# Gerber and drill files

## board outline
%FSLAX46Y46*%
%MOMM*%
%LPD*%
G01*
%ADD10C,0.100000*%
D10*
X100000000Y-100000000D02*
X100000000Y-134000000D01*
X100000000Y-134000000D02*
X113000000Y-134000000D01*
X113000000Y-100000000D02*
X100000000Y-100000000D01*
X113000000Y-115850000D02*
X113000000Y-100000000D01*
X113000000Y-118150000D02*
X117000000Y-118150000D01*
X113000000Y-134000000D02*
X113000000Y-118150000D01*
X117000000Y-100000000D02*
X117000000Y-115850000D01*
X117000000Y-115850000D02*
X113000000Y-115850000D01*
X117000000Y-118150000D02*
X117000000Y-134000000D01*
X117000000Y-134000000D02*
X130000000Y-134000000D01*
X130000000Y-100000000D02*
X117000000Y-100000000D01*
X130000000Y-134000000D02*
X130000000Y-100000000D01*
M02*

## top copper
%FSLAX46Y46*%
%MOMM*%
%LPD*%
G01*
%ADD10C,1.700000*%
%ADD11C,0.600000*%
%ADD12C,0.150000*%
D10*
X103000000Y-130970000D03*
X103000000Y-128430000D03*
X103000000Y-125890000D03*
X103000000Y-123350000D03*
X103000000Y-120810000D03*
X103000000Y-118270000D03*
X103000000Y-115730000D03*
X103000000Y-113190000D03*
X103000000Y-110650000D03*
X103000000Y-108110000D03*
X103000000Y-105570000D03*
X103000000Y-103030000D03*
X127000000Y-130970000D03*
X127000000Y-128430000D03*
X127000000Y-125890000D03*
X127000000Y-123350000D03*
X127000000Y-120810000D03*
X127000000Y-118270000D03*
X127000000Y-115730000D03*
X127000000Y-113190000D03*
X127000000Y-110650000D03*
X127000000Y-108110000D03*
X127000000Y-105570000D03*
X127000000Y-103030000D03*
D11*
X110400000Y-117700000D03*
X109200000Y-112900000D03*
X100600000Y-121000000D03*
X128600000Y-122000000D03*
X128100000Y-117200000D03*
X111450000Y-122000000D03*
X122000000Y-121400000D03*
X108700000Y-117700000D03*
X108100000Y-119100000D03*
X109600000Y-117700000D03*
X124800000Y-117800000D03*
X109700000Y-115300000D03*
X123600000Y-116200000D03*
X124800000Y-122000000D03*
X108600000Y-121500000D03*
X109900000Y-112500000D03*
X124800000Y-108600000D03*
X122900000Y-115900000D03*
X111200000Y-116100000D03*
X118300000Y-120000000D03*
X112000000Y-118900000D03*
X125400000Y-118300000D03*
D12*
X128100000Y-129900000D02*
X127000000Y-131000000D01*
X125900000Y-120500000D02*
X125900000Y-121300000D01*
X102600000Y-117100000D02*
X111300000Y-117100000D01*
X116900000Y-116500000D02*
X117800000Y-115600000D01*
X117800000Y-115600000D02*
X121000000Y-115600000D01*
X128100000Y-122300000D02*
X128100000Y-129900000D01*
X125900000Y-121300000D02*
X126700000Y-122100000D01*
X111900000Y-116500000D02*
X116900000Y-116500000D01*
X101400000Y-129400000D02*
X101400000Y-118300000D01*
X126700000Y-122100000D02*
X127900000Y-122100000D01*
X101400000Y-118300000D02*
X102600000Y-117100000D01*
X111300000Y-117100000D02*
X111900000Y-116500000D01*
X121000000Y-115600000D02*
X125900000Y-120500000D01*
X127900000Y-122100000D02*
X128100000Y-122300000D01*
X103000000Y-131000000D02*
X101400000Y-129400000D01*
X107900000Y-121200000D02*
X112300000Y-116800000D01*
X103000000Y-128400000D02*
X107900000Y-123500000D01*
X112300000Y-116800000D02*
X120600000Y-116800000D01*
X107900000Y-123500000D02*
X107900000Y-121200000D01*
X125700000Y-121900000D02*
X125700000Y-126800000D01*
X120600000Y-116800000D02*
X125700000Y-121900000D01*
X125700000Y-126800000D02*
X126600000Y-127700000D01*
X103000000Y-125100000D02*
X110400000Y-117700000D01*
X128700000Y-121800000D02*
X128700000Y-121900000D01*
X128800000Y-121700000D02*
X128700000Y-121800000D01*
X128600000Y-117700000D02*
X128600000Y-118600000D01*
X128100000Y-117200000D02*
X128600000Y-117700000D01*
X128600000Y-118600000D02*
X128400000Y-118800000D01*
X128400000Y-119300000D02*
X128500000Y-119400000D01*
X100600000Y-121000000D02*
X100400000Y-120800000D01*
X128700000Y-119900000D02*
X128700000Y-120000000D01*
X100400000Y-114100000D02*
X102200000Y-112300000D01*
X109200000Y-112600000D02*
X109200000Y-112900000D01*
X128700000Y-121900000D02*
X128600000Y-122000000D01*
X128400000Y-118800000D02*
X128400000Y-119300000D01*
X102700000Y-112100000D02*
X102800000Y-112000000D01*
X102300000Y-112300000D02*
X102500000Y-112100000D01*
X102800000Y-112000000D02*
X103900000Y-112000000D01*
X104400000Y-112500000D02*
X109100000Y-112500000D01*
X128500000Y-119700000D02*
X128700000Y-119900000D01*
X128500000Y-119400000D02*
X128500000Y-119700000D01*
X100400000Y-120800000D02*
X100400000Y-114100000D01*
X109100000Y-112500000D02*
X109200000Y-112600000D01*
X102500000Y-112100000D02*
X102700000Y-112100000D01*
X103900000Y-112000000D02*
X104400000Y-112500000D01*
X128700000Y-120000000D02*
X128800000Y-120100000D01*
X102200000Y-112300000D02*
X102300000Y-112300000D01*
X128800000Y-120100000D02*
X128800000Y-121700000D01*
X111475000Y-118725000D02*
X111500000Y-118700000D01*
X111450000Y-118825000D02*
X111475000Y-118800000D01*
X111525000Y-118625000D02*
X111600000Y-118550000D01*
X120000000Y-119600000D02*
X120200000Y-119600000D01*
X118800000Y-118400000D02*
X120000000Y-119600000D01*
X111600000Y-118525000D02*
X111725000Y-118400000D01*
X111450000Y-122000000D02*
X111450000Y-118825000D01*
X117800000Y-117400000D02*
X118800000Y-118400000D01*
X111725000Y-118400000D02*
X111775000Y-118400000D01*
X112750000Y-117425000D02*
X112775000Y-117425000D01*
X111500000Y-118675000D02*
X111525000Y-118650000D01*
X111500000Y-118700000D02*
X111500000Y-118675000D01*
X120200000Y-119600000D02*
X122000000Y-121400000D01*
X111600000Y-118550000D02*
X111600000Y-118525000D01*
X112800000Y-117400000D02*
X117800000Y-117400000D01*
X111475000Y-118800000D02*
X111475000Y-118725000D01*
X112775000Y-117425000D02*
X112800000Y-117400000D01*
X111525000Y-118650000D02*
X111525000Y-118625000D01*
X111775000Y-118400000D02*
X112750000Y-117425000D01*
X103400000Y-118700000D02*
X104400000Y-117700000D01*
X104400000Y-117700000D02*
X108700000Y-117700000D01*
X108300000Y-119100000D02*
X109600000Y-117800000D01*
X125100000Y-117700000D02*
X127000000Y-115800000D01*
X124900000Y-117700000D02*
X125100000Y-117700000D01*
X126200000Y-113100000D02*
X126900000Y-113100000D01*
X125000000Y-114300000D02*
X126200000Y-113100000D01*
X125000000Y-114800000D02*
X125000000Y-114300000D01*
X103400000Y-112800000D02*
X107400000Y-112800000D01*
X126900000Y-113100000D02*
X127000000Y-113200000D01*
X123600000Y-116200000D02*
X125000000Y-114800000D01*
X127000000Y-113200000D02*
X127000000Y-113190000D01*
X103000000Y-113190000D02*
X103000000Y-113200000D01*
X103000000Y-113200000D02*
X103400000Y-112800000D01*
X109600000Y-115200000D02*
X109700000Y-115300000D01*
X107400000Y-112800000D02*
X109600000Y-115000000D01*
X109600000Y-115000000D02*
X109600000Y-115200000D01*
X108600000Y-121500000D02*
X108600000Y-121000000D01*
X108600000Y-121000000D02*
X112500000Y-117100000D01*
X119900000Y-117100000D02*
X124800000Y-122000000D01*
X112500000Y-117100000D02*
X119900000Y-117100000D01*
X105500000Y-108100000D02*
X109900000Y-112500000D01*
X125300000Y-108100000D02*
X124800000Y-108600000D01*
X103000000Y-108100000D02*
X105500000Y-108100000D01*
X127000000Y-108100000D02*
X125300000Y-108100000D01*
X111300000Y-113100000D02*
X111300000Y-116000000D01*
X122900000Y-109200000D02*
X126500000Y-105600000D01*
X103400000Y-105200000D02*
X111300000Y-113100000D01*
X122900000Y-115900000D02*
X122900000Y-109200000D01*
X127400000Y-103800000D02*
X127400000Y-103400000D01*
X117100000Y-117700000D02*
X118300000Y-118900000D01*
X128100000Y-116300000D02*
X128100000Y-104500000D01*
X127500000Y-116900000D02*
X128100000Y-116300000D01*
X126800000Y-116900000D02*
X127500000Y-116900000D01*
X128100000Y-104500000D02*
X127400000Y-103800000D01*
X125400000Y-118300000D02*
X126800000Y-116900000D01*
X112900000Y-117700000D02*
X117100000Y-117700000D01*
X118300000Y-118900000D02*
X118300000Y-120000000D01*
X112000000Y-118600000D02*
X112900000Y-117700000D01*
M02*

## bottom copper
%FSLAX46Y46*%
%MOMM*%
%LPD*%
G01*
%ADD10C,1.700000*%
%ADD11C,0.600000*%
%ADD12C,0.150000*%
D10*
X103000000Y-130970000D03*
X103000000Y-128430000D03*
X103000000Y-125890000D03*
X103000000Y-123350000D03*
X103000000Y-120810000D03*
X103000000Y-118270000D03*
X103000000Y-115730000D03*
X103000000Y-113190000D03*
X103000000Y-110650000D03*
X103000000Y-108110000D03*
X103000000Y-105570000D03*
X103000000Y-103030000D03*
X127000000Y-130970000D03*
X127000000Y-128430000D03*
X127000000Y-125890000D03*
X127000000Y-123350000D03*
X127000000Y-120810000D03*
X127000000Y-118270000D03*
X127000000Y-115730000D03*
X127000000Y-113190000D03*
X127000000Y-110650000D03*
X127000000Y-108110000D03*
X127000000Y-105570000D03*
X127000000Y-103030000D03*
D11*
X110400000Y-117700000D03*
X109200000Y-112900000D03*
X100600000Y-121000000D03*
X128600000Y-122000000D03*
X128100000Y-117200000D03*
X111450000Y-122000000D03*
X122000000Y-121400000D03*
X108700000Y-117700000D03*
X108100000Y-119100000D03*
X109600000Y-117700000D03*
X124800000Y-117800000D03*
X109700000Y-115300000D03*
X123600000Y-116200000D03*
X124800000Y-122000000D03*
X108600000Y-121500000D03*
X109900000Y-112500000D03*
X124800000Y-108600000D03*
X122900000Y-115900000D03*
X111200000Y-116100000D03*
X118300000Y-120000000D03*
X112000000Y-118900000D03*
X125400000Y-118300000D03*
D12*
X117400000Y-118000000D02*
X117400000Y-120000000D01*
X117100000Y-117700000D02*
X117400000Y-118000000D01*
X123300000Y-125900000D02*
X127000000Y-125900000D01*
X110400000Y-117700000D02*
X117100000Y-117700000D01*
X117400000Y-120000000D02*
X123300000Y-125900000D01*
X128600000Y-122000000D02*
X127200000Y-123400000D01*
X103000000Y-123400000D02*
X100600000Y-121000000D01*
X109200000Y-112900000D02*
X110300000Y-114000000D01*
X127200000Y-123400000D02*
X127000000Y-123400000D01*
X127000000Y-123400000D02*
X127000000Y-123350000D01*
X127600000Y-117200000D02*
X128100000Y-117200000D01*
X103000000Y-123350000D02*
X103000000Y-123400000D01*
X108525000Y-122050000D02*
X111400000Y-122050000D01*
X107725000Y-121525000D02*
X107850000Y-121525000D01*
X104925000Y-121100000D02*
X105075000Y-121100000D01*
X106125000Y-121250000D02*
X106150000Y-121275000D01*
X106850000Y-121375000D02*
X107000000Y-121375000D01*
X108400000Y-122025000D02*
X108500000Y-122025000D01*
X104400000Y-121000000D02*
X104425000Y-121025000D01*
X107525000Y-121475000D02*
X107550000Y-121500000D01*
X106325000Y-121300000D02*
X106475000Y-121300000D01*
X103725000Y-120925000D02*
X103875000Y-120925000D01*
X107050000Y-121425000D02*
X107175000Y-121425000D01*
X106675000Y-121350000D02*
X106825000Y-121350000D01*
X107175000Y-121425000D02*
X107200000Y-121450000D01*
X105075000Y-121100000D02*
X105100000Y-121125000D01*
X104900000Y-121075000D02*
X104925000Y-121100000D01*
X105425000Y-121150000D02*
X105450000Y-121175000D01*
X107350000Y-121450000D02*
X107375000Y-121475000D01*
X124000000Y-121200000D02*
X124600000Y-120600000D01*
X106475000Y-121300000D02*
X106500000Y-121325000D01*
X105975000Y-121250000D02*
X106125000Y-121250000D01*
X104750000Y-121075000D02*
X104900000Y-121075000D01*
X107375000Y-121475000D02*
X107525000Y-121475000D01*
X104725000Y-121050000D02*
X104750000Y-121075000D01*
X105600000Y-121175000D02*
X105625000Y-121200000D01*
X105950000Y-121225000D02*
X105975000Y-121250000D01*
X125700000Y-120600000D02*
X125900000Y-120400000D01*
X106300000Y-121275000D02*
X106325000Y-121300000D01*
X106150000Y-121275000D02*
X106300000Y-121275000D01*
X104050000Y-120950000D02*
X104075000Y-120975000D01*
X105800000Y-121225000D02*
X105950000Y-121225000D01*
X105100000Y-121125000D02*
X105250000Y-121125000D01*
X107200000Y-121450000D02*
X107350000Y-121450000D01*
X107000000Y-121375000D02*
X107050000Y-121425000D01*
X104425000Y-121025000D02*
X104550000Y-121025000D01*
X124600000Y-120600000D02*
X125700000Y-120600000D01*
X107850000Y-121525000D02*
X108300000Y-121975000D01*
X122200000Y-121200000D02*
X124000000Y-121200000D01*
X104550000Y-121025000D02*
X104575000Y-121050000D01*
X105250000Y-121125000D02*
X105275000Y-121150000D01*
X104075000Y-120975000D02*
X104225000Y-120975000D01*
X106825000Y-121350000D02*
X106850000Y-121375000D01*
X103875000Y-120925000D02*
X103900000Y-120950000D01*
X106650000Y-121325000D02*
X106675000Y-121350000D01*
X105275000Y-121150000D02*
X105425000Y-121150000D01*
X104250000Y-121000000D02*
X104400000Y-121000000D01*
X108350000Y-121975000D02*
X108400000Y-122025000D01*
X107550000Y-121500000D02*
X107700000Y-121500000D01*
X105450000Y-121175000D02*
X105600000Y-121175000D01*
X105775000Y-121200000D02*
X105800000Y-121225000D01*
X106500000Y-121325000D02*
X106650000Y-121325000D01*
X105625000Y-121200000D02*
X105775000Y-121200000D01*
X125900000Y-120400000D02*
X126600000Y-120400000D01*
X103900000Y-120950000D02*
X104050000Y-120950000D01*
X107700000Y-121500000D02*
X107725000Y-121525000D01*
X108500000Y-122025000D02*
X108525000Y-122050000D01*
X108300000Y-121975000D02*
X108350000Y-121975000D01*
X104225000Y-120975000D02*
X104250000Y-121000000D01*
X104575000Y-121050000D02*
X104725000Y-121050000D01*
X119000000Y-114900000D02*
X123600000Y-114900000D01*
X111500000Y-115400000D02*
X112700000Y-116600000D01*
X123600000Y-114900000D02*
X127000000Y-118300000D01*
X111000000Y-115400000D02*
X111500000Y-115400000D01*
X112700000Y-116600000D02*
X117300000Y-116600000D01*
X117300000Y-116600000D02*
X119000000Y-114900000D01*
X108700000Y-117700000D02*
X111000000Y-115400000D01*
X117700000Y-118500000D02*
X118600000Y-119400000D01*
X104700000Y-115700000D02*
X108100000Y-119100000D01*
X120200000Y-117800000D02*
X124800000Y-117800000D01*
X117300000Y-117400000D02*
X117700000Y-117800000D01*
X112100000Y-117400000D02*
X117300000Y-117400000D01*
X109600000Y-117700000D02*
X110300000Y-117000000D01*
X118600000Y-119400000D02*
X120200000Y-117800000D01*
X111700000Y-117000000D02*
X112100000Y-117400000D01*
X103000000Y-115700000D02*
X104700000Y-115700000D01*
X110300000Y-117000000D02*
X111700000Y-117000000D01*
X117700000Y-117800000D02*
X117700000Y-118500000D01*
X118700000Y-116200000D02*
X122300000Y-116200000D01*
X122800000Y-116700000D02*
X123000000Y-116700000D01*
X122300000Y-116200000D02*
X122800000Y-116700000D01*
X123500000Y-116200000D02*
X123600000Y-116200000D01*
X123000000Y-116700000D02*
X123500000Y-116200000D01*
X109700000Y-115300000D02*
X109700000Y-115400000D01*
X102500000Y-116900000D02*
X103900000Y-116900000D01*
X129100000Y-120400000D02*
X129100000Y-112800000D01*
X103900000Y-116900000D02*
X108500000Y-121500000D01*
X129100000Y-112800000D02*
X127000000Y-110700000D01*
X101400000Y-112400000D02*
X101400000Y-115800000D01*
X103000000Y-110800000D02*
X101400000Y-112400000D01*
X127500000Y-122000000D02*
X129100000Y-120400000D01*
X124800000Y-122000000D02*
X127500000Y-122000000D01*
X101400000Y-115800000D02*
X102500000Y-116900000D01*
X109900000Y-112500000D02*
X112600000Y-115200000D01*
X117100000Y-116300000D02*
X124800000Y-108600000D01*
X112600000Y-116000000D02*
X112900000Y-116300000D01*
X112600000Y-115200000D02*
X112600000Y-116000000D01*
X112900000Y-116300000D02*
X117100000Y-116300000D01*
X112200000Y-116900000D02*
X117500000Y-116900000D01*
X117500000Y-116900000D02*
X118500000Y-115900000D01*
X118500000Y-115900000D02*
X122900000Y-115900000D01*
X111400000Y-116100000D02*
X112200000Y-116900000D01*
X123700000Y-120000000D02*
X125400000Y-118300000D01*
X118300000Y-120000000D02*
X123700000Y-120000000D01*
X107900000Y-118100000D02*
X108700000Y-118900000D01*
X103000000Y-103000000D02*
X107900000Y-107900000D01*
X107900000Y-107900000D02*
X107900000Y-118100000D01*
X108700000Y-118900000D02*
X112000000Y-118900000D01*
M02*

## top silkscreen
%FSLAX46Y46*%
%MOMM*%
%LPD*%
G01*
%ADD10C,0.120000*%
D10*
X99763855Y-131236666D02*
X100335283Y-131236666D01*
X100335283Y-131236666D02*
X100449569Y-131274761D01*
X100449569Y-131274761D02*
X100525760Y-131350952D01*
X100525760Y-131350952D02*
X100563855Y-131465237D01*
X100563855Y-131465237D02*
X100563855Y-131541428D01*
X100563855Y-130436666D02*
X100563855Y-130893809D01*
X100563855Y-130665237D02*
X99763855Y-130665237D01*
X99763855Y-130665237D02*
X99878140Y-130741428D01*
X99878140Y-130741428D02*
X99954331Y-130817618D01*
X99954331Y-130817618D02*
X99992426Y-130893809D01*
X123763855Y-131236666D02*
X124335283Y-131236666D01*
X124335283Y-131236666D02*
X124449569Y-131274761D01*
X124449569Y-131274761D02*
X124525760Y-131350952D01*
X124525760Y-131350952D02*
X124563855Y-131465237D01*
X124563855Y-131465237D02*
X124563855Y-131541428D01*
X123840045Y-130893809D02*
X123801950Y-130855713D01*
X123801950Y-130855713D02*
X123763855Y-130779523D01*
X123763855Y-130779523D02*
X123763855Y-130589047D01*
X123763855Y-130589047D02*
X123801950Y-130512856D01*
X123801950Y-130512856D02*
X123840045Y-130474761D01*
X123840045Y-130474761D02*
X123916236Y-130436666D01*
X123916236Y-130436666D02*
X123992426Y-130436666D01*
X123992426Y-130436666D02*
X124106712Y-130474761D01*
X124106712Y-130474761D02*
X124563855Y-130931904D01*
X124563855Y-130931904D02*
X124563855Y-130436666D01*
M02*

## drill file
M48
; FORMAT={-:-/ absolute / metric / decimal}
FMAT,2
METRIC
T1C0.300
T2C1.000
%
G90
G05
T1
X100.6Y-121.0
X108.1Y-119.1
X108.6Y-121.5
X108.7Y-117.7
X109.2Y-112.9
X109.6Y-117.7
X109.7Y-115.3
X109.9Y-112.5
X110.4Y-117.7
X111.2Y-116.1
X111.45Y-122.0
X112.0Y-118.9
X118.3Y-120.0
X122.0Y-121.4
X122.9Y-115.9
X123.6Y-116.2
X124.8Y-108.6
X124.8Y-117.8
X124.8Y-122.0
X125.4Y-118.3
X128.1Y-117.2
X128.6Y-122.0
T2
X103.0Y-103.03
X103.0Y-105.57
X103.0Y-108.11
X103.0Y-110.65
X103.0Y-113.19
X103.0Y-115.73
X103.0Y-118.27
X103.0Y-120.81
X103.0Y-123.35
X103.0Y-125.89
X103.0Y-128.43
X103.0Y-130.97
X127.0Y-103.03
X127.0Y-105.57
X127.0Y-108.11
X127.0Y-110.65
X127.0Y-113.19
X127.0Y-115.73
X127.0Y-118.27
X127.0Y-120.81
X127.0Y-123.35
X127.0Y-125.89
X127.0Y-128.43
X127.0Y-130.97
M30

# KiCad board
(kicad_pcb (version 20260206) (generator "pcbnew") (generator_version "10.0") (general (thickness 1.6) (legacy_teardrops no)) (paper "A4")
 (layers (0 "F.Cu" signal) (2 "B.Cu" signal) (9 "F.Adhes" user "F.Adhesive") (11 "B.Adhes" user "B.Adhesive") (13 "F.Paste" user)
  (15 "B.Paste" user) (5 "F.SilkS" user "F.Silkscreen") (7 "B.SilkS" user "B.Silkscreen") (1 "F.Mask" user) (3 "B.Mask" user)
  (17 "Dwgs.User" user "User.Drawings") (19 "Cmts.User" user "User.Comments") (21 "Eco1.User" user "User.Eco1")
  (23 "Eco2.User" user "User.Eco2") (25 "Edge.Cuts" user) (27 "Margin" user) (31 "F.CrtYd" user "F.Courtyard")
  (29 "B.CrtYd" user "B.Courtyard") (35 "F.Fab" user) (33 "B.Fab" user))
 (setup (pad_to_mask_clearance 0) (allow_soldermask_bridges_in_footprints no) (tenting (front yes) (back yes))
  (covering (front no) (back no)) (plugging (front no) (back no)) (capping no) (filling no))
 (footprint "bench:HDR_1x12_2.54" (layer "F.Cu") (at 103 130.97 90)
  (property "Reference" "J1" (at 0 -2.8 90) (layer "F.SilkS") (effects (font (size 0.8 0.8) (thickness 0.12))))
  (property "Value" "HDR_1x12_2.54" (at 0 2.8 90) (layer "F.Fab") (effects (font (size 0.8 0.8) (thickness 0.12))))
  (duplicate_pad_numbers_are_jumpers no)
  (pad "1" thru_hole circle (at 0 0 90) (size 1.7 1.7) (drill 1) (layers "*.Cu" "*.Mask") (remove_unused_layers no) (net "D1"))
  (pad "2" thru_hole circle (at 2.54 0 90) (size 1.7 1.7) (drill 1) (layers "*.Cu" "*.Mask") (remove_unused_layers no) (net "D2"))
  (pad "3" thru_hole circle (at 5.08 0 90) (size 1.7 1.7) (drill 1) (layers "*.Cu" "*.Mask") (remove_unused_layers no) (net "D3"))
  (pad "4" thru_hole circle (at 7.62 0 90) (size 1.7 1.7) (drill 1) (layers "*.Cu" "*.Mask") (remove_unused_layers no) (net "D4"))
  (pad "5" thru_hole circle (at 10.16 0 90) (size 1.7 1.7) (drill 1) (layers "*.Cu" "*.Mask") (remove_unused_layers no) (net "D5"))
  (pad "6" thru_hole circle (at 12.7 0 90) (size 1.7 1.7) (drill 1) (layers "*.Cu" "*.Mask") (remove_unused_layers no) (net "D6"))
  (pad "7" thru_hole circle (at 15.24 0 90) (size 1.7 1.7) (drill 1) (layers "*.Cu" "*.Mask") (remove_unused_layers no) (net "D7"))
  (pad "8" thru_hole circle (at 17.78 0 90) (size 1.7 1.7) (drill 1) (layers "*.Cu" "*.Mask") (remove_unused_layers no) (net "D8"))
  (pad "9" thru_hole circle (at 20.32 0 90) (size 1.7 1.7) (drill 1) (layers "*.Cu" "*.Mask") (remove_unused_layers no) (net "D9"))
  (pad "10" thru_hole circle (at 22.86 0 90) (size 1.7 1.7) (drill 1) (layers "*.Cu" "*.Mask") (remove_unused_layers no) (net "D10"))
  (pad "11" thru_hole circle (at 25.4 0 90) (size 1.7 1.7) (drill 1) (layers "*.Cu" "*.Mask") (remove_unused_layers no) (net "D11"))
  (pad "12" thru_hole circle (at 27.94 0 90) (size 1.7 1.7) (drill 1) (layers "*.Cu" "*.Mask") (remove_unused_layers no) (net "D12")))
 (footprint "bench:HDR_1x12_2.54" (layer "F.Cu") (at 127 130.97 90)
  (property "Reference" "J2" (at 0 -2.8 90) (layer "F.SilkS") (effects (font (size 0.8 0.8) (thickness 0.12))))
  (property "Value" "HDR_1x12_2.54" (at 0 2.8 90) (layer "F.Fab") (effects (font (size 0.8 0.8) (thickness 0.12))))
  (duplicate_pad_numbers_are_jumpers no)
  (pad "1" thru_hole circle (at 0 0 90) (size 1.7 1.7) (drill 1) (layers "*.Cu" "*.Mask") (remove_unused_layers no) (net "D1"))
  (pad "2" thru_hole circle (at 2.54 0 90) (size 1.7 1.7) (drill 1) (layers "*.Cu" "*.Mask") (remove_unused_layers no) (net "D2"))
  (pad "3" thru_hole circle (at 5.08 0 90) (size 1.7 1.7) (drill 1) (layers "*.Cu" "*.Mask") (remove_unused_layers no) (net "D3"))
  (pad "4" thru_hole circle (at 7.62 0 90) (size 1.7 1.7) (drill 1) (layers "*.Cu" "*.Mask") (remove_unused_layers no) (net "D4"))
  (pad "5" thru_hole circle (at 10.16 0 90) (size 1.7 1.7) (drill 1) (layers "*.Cu" "*.Mask") (remove_unused_layers no) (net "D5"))
  (pad "6" thru_hole circle (at 12.7 0 90) (size 1.7 1.7) (drill 1) (layers "*.Cu" "*.Mask") (remove_unused_layers no) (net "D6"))
  (pad "7" thru_hole circle (at 15.24 0 90) (size 1.7 1.7) (drill 1) (layers "*.Cu" "*.Mask") (remove_unused_layers no) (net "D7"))
  (pad "8" thru_hole circle (at 17.78 0 90) (size 1.7 1.7) (drill 1) (layers "*.Cu" "*.Mask") (remove_unused_layers no) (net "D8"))
  (pad "9" thru_hole circle (at 20.32 0 90) (size 1.7 1.7) (drill 1) (layers "*.Cu" "*.Mask") (remove_unused_layers no) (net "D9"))
  (pad "10" thru_hole circle (at 22.86 0 90) (size 1.7 1.7) (drill 1) (layers "*.Cu" "*.Mask") (remove_unused_layers no) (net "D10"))
  (pad "11" thru_hole circle (at 25.4 0 90) (size 1.7 1.7) (drill 1) (layers "*.Cu" "*.Mask") (remove_unused_layers no) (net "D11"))
  (pad "12" thru_hole circle (at 27.94 0 90) (size 1.7 1.7) (drill 1) (layers "*.Cu" "*.Mask") (remove_unused_layers no) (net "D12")))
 (gr_line (start 100 100) (end 100 134) (stroke (width 0.1) (type solid)) (layer "Edge.Cuts"))
 (gr_line (start 100 134) (end 113 134) (stroke (width 0.1) (type solid)) (layer "Edge.Cuts"))
 (gr_line (start 113 100) (end 100 100) (stroke (width 0.1) (type solid)) (layer "Edge.Cuts"))
 (gr_line (start 113 115.85) (end 113 100) (stroke (width 0.1) (type solid)) (layer "Edge.Cuts"))
 (gr_line (start 113 118.15) (end 117 118.15) (stroke (width 0.1) (type solid)) (layer "Edge.Cuts"))
 (gr_line (start 113 134) (end 113 118.15) (stroke (width 0.1) (type solid)) (layer "Edge.Cuts"))
 (gr_line (start 117 100) (end 117 115.85) (stroke (width 0.1) (type solid)) (layer "Edge.Cuts"))
 (gr_line (start 117 115.85) (end 113 115.85) (stroke (width 0.1) (type solid)) (layer "Edge.Cuts"))
 (gr_line (start 117 118.15) (end 117 134) (stroke (width 0.1) (type solid)) (layer "Edge.Cuts"))
 (gr_line (start 117 134) (end 130 134) (stroke (width 0.1) (type solid)) (layer "Edge.Cuts"))
 (gr_line (start 130 100) (end 117 100) (stroke (width 0.1) (type solid)) (layer "Edge.Cuts"))
 (gr_line (start 130 134) (end 130 100) (stroke (width 0.1) (type solid)) (layer "Edge.Cuts"))
 (segment (start 128.1 129.9) (end 127 131) (width 0.15) (layer "F.Cu") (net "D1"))
 (segment (start 125.9 120.5) (end 125.9 121.3) (width 0.15) (layer "F.Cu") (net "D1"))
 (segment (start 102.6 117.1) (end 111.3 117.1) (width 0.15) (layer "F.Cu") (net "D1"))
 (segment (start 116.9 116.5) (end 117.8 115.6) (width 0.15) (layer "F.Cu") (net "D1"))
 (segment (start 117.8 115.6) (end 121 115.6) (width 0.15) (layer "F.Cu") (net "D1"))
 (segment (start 128.1 122.3) (end 128.1 129.9) (width 0.15) (layer "F.Cu") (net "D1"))
 (segment (start 125.9 121.3) (end 126.7 122.1) (width 0.15) (layer "F.Cu") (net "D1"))
 (segment (start 111.9 116.5) (end 116.9 116.5) (width 0.15) (layer "F.Cu") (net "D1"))
 (segment (start 101.4 129.4) (end 101.4 118.3) (width 0.15) (layer "F.Cu") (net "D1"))
 (segment (start 126.7 122.1) (end 127.9 122.1) (width 0.15) (layer "F.Cu") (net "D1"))
 (segment (start 101.4 118.3) (end 102.6 117.1) (width 0.15) (layer "F.Cu") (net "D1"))
 (segment (start 111.3 117.1) (end 111.9 116.5) (width 0.15) (layer "F.Cu") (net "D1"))
 (segment (start 121 115.6) (end 125.9 120.5) (width 0.15) (layer "F.Cu") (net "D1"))
 (segment (start 127.9 122.1) (end 128.1 122.3) (width 0.15) (layer "F.Cu") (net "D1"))
 (segment (start 103 131) (end 101.4 129.4) (width 0.15) (layer "F.Cu") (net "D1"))
 (segment (start 107.9 121.2) (end 112.3 116.8) (width 0.15) (layer "F.Cu") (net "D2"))
 (segment (start 103 128.4) (end 107.9 123.5) (width 0.15) (layer "F.Cu") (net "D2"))
 (segment (start 112.3 116.8) (end 120.6 116.8) (width 0.15) (layer "F.Cu") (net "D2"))
 (segment (start 107.9 123.5) (end 107.9 121.2) (width 0.15) (layer "F.Cu") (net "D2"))
 (segment (start 125.7 121.9) (end 125.7 126.8) (width 0.15) (layer "F.Cu") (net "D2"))
 (segment (start 120.6 116.8) (end 125.7 121.9) (width 0.15) (layer "F.Cu") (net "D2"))
 (segment (start 125.7 126.8) (end 126.6 127.7) (width 0.15) (layer "F.Cu") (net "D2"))
 (segment (start 103 125.1) (end 110.4 117.7) (width 0.15) (layer "F.Cu") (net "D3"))
 (via (at 110.4 117.7) (size 0.6) (drill 0.3) (layers "F.Cu" "B.Cu") (capping no) (covering (front no) (back no))
  (plugging (front no) (back no)) (filling no) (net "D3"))
 (segment (start 117.4 118) (end 117.4 120) (width 0.15) (layer "B.Cu") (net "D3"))
 (segment (start 117.1 117.7) (end 117.4 118) (width 0.15) (layer "B.Cu") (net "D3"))
 (segment (start 123.3 125.9) (end 127 125.9) (width 0.15) (layer "B.Cu") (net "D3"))
 (segment (start 110.4 117.7) (end 117.1 117.7) (width 0.15) (layer "B.Cu") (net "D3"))
 (segment (start 117.4 120) (end 123.3 125.9) (width 0.15) (layer "B.Cu") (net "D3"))
 (segment (start 128.7 121.8) (end 128.7 121.9) (width 0.15) (layer "F.Cu") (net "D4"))
 (segment (start 128.8 121.7) (end 128.7 121.8) (width 0.15) (layer "F.Cu") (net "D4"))
 (segment (start 128.6 117.7) (end 128.6 118.6) (width 0.15) (layer "F.Cu") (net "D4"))
 (segment (start 128.1 117.2) (end 128.6 117.7) (width 0.15) (layer "F.Cu") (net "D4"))
 (segment (start 128.6 118.6) (end 128.4 118.8) (width 0.15) (layer "F.Cu") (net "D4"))
 (segment (start 128.4 119.3) (end 128.5 119.4) (width 0.15) (layer "F.Cu") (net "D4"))
 (segment (start 100.6 121) (end 100.4 120.8) (width 0.15) (layer "F.Cu") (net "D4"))
 (segment (start 128.7 119.9) (end 128.7 120) (width 0.15) (layer "F.Cu") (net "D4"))
 (segment (start 100.4 114.1) (end 102.2 112.3) (width 0.15) (layer "F.Cu") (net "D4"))
 (segment (start 109.2 112.6) (end 109.2 112.9) (width 0.15) (layer "F.Cu") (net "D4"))
 (segment (start 128.7 121.9) (end 128.6 122) (width 0.15) (layer "F.Cu") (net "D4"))
 (segment (start 128.4 118.8) (end 128.4 119.3) (width 0.15) (layer "F.Cu") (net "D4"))
 (segment (start 102.7 112.1) (end 102.8 112) (width 0.15) (layer "F.Cu") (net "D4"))
 (segment (start 102.3 112.3) (end 102.5 112.1) (width 0.15) (layer "F.Cu") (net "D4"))
 (segment (start 102.8 112) (end 103.9 112) (width 0.15) (layer "F.Cu") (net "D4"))
 (segment (start 104.4 112.5) (end 109.1 112.5) (width 0.15) (layer "F.Cu") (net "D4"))
 (segment (start 128.5 119.7) (end 128.7 119.9) (width 0.15) (layer "F.Cu") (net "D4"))
 (segment (start 128.5 119.4) (end 128.5 119.7) (width 0.15) (layer "F.Cu") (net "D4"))
 (segment (start 100.4 120.8) (end 100.4 114.1) (width 0.15) (layer "F.Cu") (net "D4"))
 (segment (start 109.1 112.5) (end 109.2 112.6) (width 0.15) (layer "F.Cu") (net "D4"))
 (segment (start 102.5 112.1) (end 102.7 112.1) (width 0.15) (layer "F.Cu") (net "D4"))
 (segment (start 103.9 112) (end 104.4 112.5) (width 0.15) (layer "F.Cu") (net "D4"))
 (segment (start 128.7 120) (end 128.8 120.1) (width 0.15) (layer "F.Cu") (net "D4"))
 (segment (start 102.2 112.3) (end 102.3 112.3) (width 0.15) (layer "F.Cu") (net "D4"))
 (segment (start 128.8 120.1) (end 128.8 121.7) (width 0.15) (layer "F.Cu") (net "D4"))
 (via (at 109.2 112.9) (size 0.6) (drill 0.3) (layers "F.Cu" "B.Cu") (capping no) (covering (front no) (back no))
  (plugging (front no) (back no)) (filling no) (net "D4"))
 (via (at 100.6 121) (size 0.6) (drill 0.3) (layers "F.Cu" "B.Cu") (capping no) (covering (front no) (back no))
  (plugging (front no) (back no)) (filling no) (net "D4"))
 (via (at 128.6 122) (size 0.6) (drill 0.3) (layers "F.Cu" "B.Cu") (capping no) (covering (front no) (back no))
  (plugging (front no) (back no)) (filling no) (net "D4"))
 (via (at 128.1 117.2) (size 0.6) (drill 0.3) (layers "F.Cu" "B.Cu") (capping no) (covering (front no) (back no))
  (plugging (front no) (back no)) (filling no) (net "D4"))
 (segment (start 128.6 122) (end 127.2 123.4) (width 0.15) (layer "B.Cu") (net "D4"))
 (segment (start 103 123.4) (end 100.6 121) (width 0.15) (layer "B.Cu") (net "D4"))
 (segment (start 109.2 112.9) (end 110.3 114) (width 0.15) (layer "B.Cu") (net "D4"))
 (segment (start 127.2 123.4) (end 127 123.4) (width 0.15) (layer "B.Cu") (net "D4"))
 (segment (start 127 123.4) (end 127 123.35) (width 0.15) (layer "B.Cu") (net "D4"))
 (segment (start 127.6 117.2) (end 128.1 117.2) (width 0.15) (layer "B.Cu") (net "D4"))
 (segment (start 103 123.35) (end 103 123.4) (width 0.15) (layer "B.Cu") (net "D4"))
 (segment (start 111.475 118.725) (end 111.5 118.7) (width 0.15) (layer "F.Cu") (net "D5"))
 (segment (start 111.45 118.825) (end 111.475 118.8) (width 0.15) (layer "F.Cu") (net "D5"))
 (segment (start 111.525 118.625) (end 111.6 118.55) (width 0.15) (layer "F.Cu") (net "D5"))
 (segment (start 120 119.6) (end 120.2 119.6) (width 0.15) (layer "F.Cu") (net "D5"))
 (segment (start 118.8 118.4) (end 120 119.6) (width 0.15) (layer "F.Cu") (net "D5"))
 (segment (start 111.6 118.525) (end 111.725 118.4) (width 0.15) (layer "F.Cu") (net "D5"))
 (segment (start 111.45 122) (end 111.45 118.825) (width 0.15) (layer "F.Cu") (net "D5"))
 (segment (start 117.8 117.4) (end 118.8 118.4) (width 0.15) (layer "F.Cu") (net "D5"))
 (segment (start 111.725 118.4) (end 111.775 118.4) (width 0.15) (layer "F.Cu") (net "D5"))
 (segment (start 112.75 117.425) (end 112.775 117.425) (width 0.15) (layer "F.Cu") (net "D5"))
 (segment (start 111.5 118.675) (end 111.525 118.65) (width 0.15) (layer "F.Cu") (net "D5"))
 (segment (start 111.5 118.7) (end 111.5 118.675) (width 0.15) (layer "F.Cu") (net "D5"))
 (segment (start 120.2 119.6) (end 122 121.4) (width 0.15) (layer "F.Cu") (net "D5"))
 (segment (start 111.6 118.55) (end 111.6 118.525) (width 0.15) (layer "F.Cu") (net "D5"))
 (segment (start 112.8 117.4) (end 117.8 117.4) (width 0.15) (layer "F.Cu") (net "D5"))
 (segment (start 111.475 118.8) (end 111.475 118.725) (width 0.15) (layer "F.Cu") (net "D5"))
 (segment (start 112.775 117.425) (end 112.8 117.4) (width 0.15) (layer "F.Cu") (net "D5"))
 (segment (start 111.525 118.65) (end 111.525 118.625) (width 0.15) (layer "F.Cu") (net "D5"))
 (segment (start 111.775 118.4) (end 112.75 117.425) (width 0.15) (layer "F.Cu") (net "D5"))
 (via (at 111.45 122) (size 0.6) (drill 0.3) (layers "F.Cu" "B.Cu") (capping no) (covering (front no) (back no))
  (plugging (front no) (back no)) (filling no) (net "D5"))
 (via (at 122 121.4) (size 0.6) (drill 0.3) (layers "F.Cu" "B.Cu") (capping no) (covering (front no) (back no))
  (plugging (front no) (back no)) (filling no) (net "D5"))
 (segment (start 108.525 122.05) (end 111.4 122.05) (width 0.15) (layer "B.Cu") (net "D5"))
 (segment (start 107.725 121.525) (end 107.85 121.525) (width 0.15) (layer "B.Cu") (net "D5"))
 (segment (start 104.925 121.1) (end 105.075 121.1) (width 0.15) (layer "B.Cu") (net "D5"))
 (segment (start 106.125 121.25) (end 106.15 121.275) (width 0.15) (layer "B.Cu") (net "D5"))
 (segment (start 106.85 121.375) (end 107 121.375) (width 0.15) (layer "B.Cu") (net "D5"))
 (segment (start 108.4 122.025) (end 108.5 122.025) (width 0.15) (layer "B.Cu") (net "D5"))
 (segment (start 104.4 121) (end 104.425 121.025) (width 0.15) (layer "B.Cu") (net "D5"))
 (segment (start 107.525 121.475) (end 107.55 121.5) (width 0.15) (layer "B.Cu") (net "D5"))
 (segment (start 106.325 121.3) (end 106.475 121.3) (width 0.15) (layer "B.Cu") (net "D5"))
 (segment (start 103.725 120.925) (end 103.875 120.925) (width 0.15) (layer "B.Cu") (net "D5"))
 (segment (start 107.05 121.425) (end 107.175 121.425) (width 0.15) (layer "B.Cu") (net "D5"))
 (segment (start 106.675 121.35) (end 106.825 121.35) (width 0.15) (layer "B.Cu") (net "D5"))
 (segment (start 107.175 121.425) (end 107.2 121.45) (width 0.15) (layer "B.Cu") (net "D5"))
 (segment (start 105.075 121.1) (end 105.1 121.125) (width 0.15) (layer "B.Cu") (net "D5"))
 (segment (start 104.9 121.075) (end 104.925 121.1) (width 0.15) (layer "B.Cu") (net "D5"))
 (segment (start 105.425 121.15) (end 105.45 121.175) (width 0.15) (layer "B.Cu") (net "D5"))
 (segment (start 107.35 121.45) (end 107.375 121.475) (width 0.15) (layer "B.Cu") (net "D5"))
 (segment (start 124 121.2) (end 124.6 120.6) (width 0.15) (layer "B.Cu") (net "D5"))
 (segment (start 106.475 121.3) (end 106.5 121.325) (width 0.15) (layer "B.Cu") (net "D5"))
 (segment (start 105.975 121.25) (end 106.125 121.25) (width 0.15) (layer "B.Cu") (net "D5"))
 (segment (start 104.75 121.075) (end 104.9 121.075) (width 0.15) (layer "B.Cu") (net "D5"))
 (segment (start 107.375 121.475) (end 107.525 121.475) (width 0.15) (layer "B.Cu") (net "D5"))
 (segment (start 104.725 121.05) (end 104.75 121.075) (width 0.15) (layer "B.Cu") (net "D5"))
 (segment (start 105.6 121.175) (end 105.625 121.2) (width 0.15) (layer "B.Cu") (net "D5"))
 (segment (start 105.95 121.225) (end 105.975 121.25) (width 0.15) (layer "B.Cu") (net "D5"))
 (segment (start 125.7 120.6) (end 125.9 120.4) (width 0.15) (layer "B.Cu") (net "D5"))
 (segment (start 106.3 121.275) (end 106.325 121.3) (width 0.15) (layer "B.Cu") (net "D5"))
 (segment (start 106.15 121.275) (end 106.3 121.275) (width 0.15) (layer "B.Cu") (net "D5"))
 (segment (start 104.05 120.95) (end 104.075 120.975) (width 0.15) (layer "B.Cu") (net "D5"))
 (segment (start 105.8 121.225) (end 105.95 121.225) (width 0.15) (layer "B.Cu") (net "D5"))
 (segment (start 105.1 121.125) (end 105.25 121.125) (width 0.15) (layer "B.Cu") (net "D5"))
 (segment (start 107.2 121.45) (end 107.35 121.45) (width 0.15) (layer "B.Cu") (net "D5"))
 (segment (start 107 121.375) (end 107.05 121.425) (width 0.15) (layer "B.Cu") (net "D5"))
 (segment (start 104.425 121.025) (end 104.55 121.025) (width 0.15) (layer "B.Cu") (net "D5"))
 (segment (start 124.6 120.6) (end 125.7 120.6) (width 0.15) (layer "B.Cu") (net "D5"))
 (segment (start 107.85 121.525) (end 108.3 121.975) (width 0.15) (layer "B.Cu") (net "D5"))
 (segment (start 122.2 121.2) (end 124 121.2) (width 0.15) (layer "B.Cu") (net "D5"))
 (segment (start 104.55 121.025) (end 104.575 121.05) (width 0.15) (layer "B.Cu") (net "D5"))
 (segment (start 105.25 121.125) (end 105.275 121.15) (width 0.15) (layer "B.Cu") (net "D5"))
 (segment (start 104.075 120.975) (end 104.225 120.975) (width 0.15) (layer "B.Cu") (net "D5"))
 (segment (start 106.825 121.35) (end 106.85 121.375) (width 0.15) (layer "B.Cu") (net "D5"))
 (segment (start 103.875 120.925) (end 103.9 120.95) (width 0.15) (layer "B.Cu") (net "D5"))
 (segment (start 106.65 121.325) (end 106.675 121.35) (width 0.15) (layer "B.Cu") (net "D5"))
 (segment (start 105.275 121.15) (end 105.425 121.15) (width 0.15) (layer "B.Cu") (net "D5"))
 (segment (start 104.25 121) (end 104.4 121) (width 0.15) (layer "B.Cu") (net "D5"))
 (segment (start 108.35 121.975) (end 108.4 122.025) (width 0.15) (layer "B.Cu") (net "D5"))
 (segment (start 107.55 121.5) (end 107.7 121.5) (width 0.15) (layer "B.Cu") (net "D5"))
 (segment (start 105.45 121.175) (end 105.6 121.175) (width 0.15) (layer "B.Cu") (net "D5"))
 (segment (start 105.775 121.2) (end 105.8 121.225) (width 0.15) (layer "B.Cu") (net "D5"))
 (segment (start 106.5 121.325) (end 106.65 121.325) (width 0.15) (layer "B.Cu") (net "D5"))
 (segment (start 105.625 121.2) (end 105.775 121.2) (width 0.15) (layer "B.Cu") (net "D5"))
 (segment (start 125.9 120.4) (end 126.6 120.4) (width 0.15) (layer "B.Cu") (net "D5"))
 (segment (start 103.9 120.95) (end 104.05 120.95) (width 0.15) (layer "B.Cu") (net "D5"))
 (segment (start 107.7 121.5) (end 107.725 121.525) (width 0.15) (layer "B.Cu") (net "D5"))
 (segment (start 108.5 122.025) (end 108.525 122.05) (width 0.15) (layer "B.Cu") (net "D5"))
 (segment (start 108.3 121.975) (end 108.35 121.975) (width 0.15) (layer "B.Cu") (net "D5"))
 (segment (start 104.225 120.975) (end 104.25 121) (width 0.15) (layer "B.Cu") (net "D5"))
 (segment (start 104.575 121.05) (end 104.725 121.05) (width 0.15) (layer "B.Cu") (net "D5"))
 (segment (start 103.4 118.7) (end 104.4 117.7) (width 0.15) (layer "F.Cu") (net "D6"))
 (segment (start 104.4 117.7) (end 108.7 117.7) (width 0.15) (layer "F.Cu") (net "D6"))
 (via (at 108.7 117.7) (size 0.6) (drill 0.3) (layers "F.Cu" "B.Cu") (capping no) (covering (front no) (back no))
  (plugging (front no) (back no)) (filling no) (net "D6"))
 (segment (start 119 114.9) (end 123.6 114.9) (width 0.15) (layer "B.Cu") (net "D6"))
 (segment (start 111.5 115.4) (end 112.7 116.6) (width 0.15) (layer "B.Cu") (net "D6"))
 (segment (start 123.6 114.9) (end 127 118.3) (width 0.15) (layer "B.Cu") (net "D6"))
 (segment (start 111 115.4) (end 111.5 115.4) (width 0.15) (layer "B.Cu") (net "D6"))
 (segment (start 112.7 116.6) (end 117.3 116.6) (width 0.15) (layer "B.Cu") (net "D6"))
 (segment (start 117.3 116.6) (end 119 114.9) (width 0.15) (layer "B.Cu") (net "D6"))
 (segment (start 108.7 117.7) (end 111 115.4) (width 0.15) (layer "B.Cu") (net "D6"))
 (segment (start 108.3 119.1) (end 109.6 117.8) (width 0.15) (layer "F.Cu") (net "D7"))
 (segment (start 125.1 117.7) (end 127 115.8) (width 0.15) (layer "F.Cu") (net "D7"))
 (segment (start 124.9 117.7) (end 125.1 117.7) (width 0.15) (layer "F.Cu") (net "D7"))
 (via (at 108.1 119.1) (size 0.6) (drill 0.3) (layers "F.Cu" "B.Cu") (capping no) (covering (front no) (back no))
  (plugging (front no) (back no)) (filling no) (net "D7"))
 (via (at 109.6 117.7) (size 0.6) (drill 0.3) (layers "F.Cu" "B.Cu") (capping no) (covering (front no) (back no))
  (plugging (front no) (back no)) (filling no) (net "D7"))
 (via (at 124.8 117.8) (size 0.6) (drill 0.3) (layers "F.Cu" "B.Cu") (capping no) (covering (front no) (back no))
  (plugging (front no) (back no)) (filling no) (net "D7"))
 (segment (start 117.7 118.5) (end 118.6 119.4) (width 0.15) (layer "B.Cu") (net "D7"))
 (segment (start 104.7 115.7) (end 108.1 119.1) (width 0.15) (layer "B.Cu") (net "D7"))
 (segment (start 120.2 117.8) (end 124.8 117.8) (width 0.15) (layer "B.Cu") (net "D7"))
 (segment (start 117.3 117.4) (end 117.7 117.8) (width 0.15) (layer "B.Cu") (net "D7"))
 (segment (start 112.1 117.4) (end 117.3 117.4) (width 0.15) (layer "B.Cu") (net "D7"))
 (segment (start 109.6 117.7) (end 110.3 117) (width 0.15) (layer "B.Cu") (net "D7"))
 (segment (start 118.6 119.4) (end 120.2 117.8) (width 0.15) (layer "B.Cu") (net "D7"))
 (segment (start 111.7 117) (end 112.1 117.4) (width 0.15) (layer "B.Cu") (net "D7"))
 (segment (start 103 115.7) (end 104.7 115.7) (width 0.15) (layer "B.Cu") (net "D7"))
 (segment (start 110.3 117) (end 111.7 117) (width 0.15) (layer "B.Cu") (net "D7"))
 (segment (start 117.7 117.8) (end 117.7 118.5) (width 0.15) (layer "B.Cu") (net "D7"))
 (segment (start 126.2 113.1) (end 126.9 113.1) (width 0.15) (layer "F.Cu") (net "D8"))
 (segment (start 125 114.3) (end 126.2 113.1) (width 0.15) (layer "F.Cu") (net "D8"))
 (segment (start 125 114.8) (end 125 114.3) (width 0.15) (layer "F.Cu") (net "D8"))
 (segment (start 103.4 112.8) (end 107.4 112.8) (width 0.15) (layer "F.Cu") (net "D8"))
 (segment (start 126.9 113.1) (end 127 113.2) (width 0.15) (layer "F.Cu") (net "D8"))
 (segment (start 123.6 116.2) (end 125 114.8) (width 0.15) (layer "F.Cu") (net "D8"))
 (segment (start 127 113.2) (end 127 113.19) (width 0.15) (layer "F.Cu") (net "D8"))
 (segment (start 103 113.19) (end 103 113.2) (width 0.15) (layer "F.Cu") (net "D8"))
 (segment (start 103 113.2) (end 103.4 112.8) (width 0.15) (layer "F.Cu") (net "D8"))
 (segment (start 109.6 115.2) (end 109.7 115.3) (width 0.15) (layer "F.Cu") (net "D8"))
 (segment (start 107.4 112.8) (end 109.6 115) (width 0.15) (layer "F.Cu") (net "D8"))
 (segment (start 109.6 115) (end 109.6 115.2) (width 0.15) (layer "F.Cu") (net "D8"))
 (via (at 109.7 115.3) (size 0.6) (drill 0.3) (layers "F.Cu" "B.Cu") (capping no) (covering (front no) (back no))
  (plugging (front no) (back no)) (filling no) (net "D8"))
 (via (at 123.6 116.2) (size 0.6) (drill 0.3) (layers "F.Cu" "B.Cu") (capping no) (covering (front no) (back no))
  (plugging (front no) (back no)) (filling no) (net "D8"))
 (segment (start 118.7 116.2) (end 122.3 116.2) (width 0.15) (layer "B.Cu") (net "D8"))
 (segment (start 122.8 116.7) (end 123 116.7) (width 0.15) (layer "B.Cu") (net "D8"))
 (segment (start 122.3 116.2) (end 122.8 116.7) (width 0.15) (layer "B.Cu") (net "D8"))
 (segment (start 123.5 116.2) (end 123.6 116.2) (width 0.15) (layer "B.Cu") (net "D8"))
 (segment (start 123 116.7) (end 123.5 116.2) (width 0.15) (layer "B.Cu") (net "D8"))
 (segment (start 109.7 115.3) (end 109.7 115.4) (width 0.15) (layer "B.Cu") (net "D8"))
 (segment (start 108.6 121.5) (end 108.6 121) (width 0.15) (layer "F.Cu") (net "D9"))
 (segment (start 108.6 121) (end 112.5 117.1) (width 0.15) (layer "F.Cu") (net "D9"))
 (segment (start 119.9 117.1) (end 124.8 122) (width 0.15) (layer "F.Cu") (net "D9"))
 (segment (start 112.5 117.1) (end 119.9 117.1) (width 0.15) (layer "F.Cu") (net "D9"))
 (via (at 124.8 122) (size 0.6) (drill 0.3) (layers "F.Cu" "B.Cu") (capping no) (covering (front no) (back no))
  (plugging (front no) (back no)) (filling no) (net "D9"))
 (via (at 108.6 121.5) (size 0.6) (drill 0.3) (layers "F.Cu" "B.Cu") (capping no) (covering (front no) (back no))
  (plugging (front no) (back no)) (filling no) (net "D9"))
 (segment (start 102.5 116.9) (end 103.9 116.9) (width 0.15) (layer "B.Cu") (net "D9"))
 (segment (start 129.1 120.4) (end 129.1 112.8) (width 0.15) (layer "B.Cu") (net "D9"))
 (segment (start 103.9 116.9) (end 108.5 121.5) (width 0.15) (layer "B.Cu") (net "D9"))
 (segment (start 129.1 112.8) (end 127 110.7) (width 0.15) (layer "B.Cu") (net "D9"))
 (segment (start 101.4 112.4) (end 101.4 115.8) (width 0.15) (layer "B.Cu") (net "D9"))
 (segment (start 103 110.8) (end 101.4 112.4) (width 0.15) (layer "B.Cu") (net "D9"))
 (segment (start 127.5 122) (end 129.1 120.4) (width 0.15) (layer "B.Cu") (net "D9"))
 (segment (start 124.8 122) (end 127.5 122) (width 0.15) (layer "B.Cu") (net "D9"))
 (segment (start 101.4 115.8) (end 102.5 116.9) (width 0.15) (layer "B.Cu") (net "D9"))
 (segment (start 105.5 108.1) (end 109.9 112.5) (width 0.15) (layer "F.Cu") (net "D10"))
 (segment (start 125.3 108.1) (end 124.8 108.6) (width 0.15) (layer "F.Cu") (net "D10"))
 (segment (start 103 108.1) (end 105.5 108.1) (width 0.15) (layer "F.Cu") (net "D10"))
 (segment (start 127 108.1) (end 125.3 108.1) (width 0.15) (layer "F.Cu") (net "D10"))
 (via (at 109.9 112.5) (size 0.6) (drill 0.3) (layers "F.Cu" "B.Cu") (capping no) (covering (front no) (back no))
  (plugging (front no) (back no)) (filling no) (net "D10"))
 (via (at 124.8 108.6) (size 0.6) (drill 0.3) (layers "F.Cu" "B.Cu") (capping no) (covering (front no) (back no))
  (plugging (front no) (back no)) (filling no) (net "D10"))
 (segment (start 109.9 112.5) (end 112.6 115.2) (width 0.15) (layer "B.Cu") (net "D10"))
 (segment (start 117.1 116.3) (end 124.8 108.6) (width 0.15) (layer "B.Cu") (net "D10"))
 (segment (start 112.6 116) (end 112.9 116.3) (width 0.15) (layer "B.Cu") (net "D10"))
 (segment (start 112.6 115.2) (end 112.6 116) (width 0.15) (layer "B.Cu") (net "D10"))
 (segment (start 112.9 116.3) (end 117.1 116.3) (width 0.15) (layer "B.Cu") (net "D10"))
 (segment (start 111.3 113.1) (end 111.3 116) (width 0.15) (layer "F.Cu") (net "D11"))
 (segment (start 122.9 109.2) (end 126.5 105.6) (width 0.15) (layer "F.Cu") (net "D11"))
 (segment (start 103.4 105.2) (end 111.3 113.1) (width 0.15) (layer "F.Cu") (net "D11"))
 (segment (start 122.9 115.9) (end 122.9 109.2) (width 0.15) (layer "F.Cu") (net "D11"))
 (via (at 122.9 115.9) (size 0.6) (drill 0.3) (layers "F.Cu" "B.Cu") (capping no) (covering (front no) (back no))
  (plugging (front no) (back no)) (filling no) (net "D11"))
 (via (at 111.2 116.1) (size 0.6) (drill 0.3) (layers "F.Cu" "B.Cu") (capping no) (covering (front no) (back no))
  (plugging (front no) (back no)) (filling no) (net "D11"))
 (segment (start 112.2 116.9) (end 117.5 116.9) (width 0.15) (layer "B.Cu") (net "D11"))
 (segment (start 117.5 116.9) (end 118.5 115.9) (width 0.15) (layer "B.Cu") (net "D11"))
 (segment (start 118.5 115.9) (end 122.9 115.9) (width 0.15) (layer "B.Cu") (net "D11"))
 (segment (start 111.4 116.1) (end 112.2 116.9) (width 0.15) (layer "B.Cu") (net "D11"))
 (segment (start 127.4 103.8) (end 127.4 103.4) (width 0.15) (layer "F.Cu") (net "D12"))
 (segment (start 117.1 117.7) (end 118.3 118.9) (width 0.15) (layer "F.Cu") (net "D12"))
 (segment (start 128.1 116.3) (end 128.1 104.5) (width 0.15) (layer "F.Cu") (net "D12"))
 (segment (start 127.5 116.9) (end 128.1 116.3) (width 0.15) (layer "F.Cu") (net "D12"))
 (segment (start 126.8 116.9) (end 127.5 116.9) (width 0.15) (layer "F.Cu") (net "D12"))
 (segment (start 128.1 104.5) (end 127.4 103.8) (width 0.15) (layer "F.Cu") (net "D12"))
 (segment (start 125.4 118.3) (end 126.8 116.9) (width 0.15) (layer "F.Cu") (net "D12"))
 (segment (start 112.9 117.7) (end 117.1 117.7) (width 0.15) (layer "F.Cu") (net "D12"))
 (segment (start 118.3 118.9) (end 118.3 120) (width 0.15) (layer "F.Cu") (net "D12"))
 (segment (start 112 118.6) (end 112.9 117.7) (width 0.15) (layer "F.Cu") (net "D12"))
 (via (at 118.3 120) (size 0.6) (drill 0.3) (layers "F.Cu" "B.Cu") (capping no) (covering (front no) (back no))
  (plugging (front no) (back no)) (filling no) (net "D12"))
 (via (at 112 118.9) (size 0.6) (drill 0.3) (layers "F.Cu" "B.Cu") (capping no) (covering (front no) (back no))
  (plugging (front no) (back no)) (filling no) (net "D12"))
 (via (at 125.4 118.3) (size 0.6) (drill 0.3) (layers "F.Cu" "B.Cu") (capping no) (covering (front no) (back no))
  (plugging (front no) (back no)) (filling no) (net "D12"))
 (segment (start 123.7 120) (end 125.4 118.3) (width 0.15) (layer "B.Cu") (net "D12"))
 (segment (start 118.3 120) (end 123.7 120) (width 0.15) (layer "B.Cu") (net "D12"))
 (segment (start 107.9 118.1) (end 108.7 118.9) (width 0.15) (layer "B.Cu") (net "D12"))
 (segment (start 103 103) (end 107.9 107.9) (width 0.15) (layer "B.Cu") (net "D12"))
 (segment (start 107.9 107.9) (end 107.9 118.1) (width 0.15) (layer "B.Cu") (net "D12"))
 (segment (start 108.7 118.9) (end 112 118.9) (width 0.15) (layer "B.Cu") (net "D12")))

